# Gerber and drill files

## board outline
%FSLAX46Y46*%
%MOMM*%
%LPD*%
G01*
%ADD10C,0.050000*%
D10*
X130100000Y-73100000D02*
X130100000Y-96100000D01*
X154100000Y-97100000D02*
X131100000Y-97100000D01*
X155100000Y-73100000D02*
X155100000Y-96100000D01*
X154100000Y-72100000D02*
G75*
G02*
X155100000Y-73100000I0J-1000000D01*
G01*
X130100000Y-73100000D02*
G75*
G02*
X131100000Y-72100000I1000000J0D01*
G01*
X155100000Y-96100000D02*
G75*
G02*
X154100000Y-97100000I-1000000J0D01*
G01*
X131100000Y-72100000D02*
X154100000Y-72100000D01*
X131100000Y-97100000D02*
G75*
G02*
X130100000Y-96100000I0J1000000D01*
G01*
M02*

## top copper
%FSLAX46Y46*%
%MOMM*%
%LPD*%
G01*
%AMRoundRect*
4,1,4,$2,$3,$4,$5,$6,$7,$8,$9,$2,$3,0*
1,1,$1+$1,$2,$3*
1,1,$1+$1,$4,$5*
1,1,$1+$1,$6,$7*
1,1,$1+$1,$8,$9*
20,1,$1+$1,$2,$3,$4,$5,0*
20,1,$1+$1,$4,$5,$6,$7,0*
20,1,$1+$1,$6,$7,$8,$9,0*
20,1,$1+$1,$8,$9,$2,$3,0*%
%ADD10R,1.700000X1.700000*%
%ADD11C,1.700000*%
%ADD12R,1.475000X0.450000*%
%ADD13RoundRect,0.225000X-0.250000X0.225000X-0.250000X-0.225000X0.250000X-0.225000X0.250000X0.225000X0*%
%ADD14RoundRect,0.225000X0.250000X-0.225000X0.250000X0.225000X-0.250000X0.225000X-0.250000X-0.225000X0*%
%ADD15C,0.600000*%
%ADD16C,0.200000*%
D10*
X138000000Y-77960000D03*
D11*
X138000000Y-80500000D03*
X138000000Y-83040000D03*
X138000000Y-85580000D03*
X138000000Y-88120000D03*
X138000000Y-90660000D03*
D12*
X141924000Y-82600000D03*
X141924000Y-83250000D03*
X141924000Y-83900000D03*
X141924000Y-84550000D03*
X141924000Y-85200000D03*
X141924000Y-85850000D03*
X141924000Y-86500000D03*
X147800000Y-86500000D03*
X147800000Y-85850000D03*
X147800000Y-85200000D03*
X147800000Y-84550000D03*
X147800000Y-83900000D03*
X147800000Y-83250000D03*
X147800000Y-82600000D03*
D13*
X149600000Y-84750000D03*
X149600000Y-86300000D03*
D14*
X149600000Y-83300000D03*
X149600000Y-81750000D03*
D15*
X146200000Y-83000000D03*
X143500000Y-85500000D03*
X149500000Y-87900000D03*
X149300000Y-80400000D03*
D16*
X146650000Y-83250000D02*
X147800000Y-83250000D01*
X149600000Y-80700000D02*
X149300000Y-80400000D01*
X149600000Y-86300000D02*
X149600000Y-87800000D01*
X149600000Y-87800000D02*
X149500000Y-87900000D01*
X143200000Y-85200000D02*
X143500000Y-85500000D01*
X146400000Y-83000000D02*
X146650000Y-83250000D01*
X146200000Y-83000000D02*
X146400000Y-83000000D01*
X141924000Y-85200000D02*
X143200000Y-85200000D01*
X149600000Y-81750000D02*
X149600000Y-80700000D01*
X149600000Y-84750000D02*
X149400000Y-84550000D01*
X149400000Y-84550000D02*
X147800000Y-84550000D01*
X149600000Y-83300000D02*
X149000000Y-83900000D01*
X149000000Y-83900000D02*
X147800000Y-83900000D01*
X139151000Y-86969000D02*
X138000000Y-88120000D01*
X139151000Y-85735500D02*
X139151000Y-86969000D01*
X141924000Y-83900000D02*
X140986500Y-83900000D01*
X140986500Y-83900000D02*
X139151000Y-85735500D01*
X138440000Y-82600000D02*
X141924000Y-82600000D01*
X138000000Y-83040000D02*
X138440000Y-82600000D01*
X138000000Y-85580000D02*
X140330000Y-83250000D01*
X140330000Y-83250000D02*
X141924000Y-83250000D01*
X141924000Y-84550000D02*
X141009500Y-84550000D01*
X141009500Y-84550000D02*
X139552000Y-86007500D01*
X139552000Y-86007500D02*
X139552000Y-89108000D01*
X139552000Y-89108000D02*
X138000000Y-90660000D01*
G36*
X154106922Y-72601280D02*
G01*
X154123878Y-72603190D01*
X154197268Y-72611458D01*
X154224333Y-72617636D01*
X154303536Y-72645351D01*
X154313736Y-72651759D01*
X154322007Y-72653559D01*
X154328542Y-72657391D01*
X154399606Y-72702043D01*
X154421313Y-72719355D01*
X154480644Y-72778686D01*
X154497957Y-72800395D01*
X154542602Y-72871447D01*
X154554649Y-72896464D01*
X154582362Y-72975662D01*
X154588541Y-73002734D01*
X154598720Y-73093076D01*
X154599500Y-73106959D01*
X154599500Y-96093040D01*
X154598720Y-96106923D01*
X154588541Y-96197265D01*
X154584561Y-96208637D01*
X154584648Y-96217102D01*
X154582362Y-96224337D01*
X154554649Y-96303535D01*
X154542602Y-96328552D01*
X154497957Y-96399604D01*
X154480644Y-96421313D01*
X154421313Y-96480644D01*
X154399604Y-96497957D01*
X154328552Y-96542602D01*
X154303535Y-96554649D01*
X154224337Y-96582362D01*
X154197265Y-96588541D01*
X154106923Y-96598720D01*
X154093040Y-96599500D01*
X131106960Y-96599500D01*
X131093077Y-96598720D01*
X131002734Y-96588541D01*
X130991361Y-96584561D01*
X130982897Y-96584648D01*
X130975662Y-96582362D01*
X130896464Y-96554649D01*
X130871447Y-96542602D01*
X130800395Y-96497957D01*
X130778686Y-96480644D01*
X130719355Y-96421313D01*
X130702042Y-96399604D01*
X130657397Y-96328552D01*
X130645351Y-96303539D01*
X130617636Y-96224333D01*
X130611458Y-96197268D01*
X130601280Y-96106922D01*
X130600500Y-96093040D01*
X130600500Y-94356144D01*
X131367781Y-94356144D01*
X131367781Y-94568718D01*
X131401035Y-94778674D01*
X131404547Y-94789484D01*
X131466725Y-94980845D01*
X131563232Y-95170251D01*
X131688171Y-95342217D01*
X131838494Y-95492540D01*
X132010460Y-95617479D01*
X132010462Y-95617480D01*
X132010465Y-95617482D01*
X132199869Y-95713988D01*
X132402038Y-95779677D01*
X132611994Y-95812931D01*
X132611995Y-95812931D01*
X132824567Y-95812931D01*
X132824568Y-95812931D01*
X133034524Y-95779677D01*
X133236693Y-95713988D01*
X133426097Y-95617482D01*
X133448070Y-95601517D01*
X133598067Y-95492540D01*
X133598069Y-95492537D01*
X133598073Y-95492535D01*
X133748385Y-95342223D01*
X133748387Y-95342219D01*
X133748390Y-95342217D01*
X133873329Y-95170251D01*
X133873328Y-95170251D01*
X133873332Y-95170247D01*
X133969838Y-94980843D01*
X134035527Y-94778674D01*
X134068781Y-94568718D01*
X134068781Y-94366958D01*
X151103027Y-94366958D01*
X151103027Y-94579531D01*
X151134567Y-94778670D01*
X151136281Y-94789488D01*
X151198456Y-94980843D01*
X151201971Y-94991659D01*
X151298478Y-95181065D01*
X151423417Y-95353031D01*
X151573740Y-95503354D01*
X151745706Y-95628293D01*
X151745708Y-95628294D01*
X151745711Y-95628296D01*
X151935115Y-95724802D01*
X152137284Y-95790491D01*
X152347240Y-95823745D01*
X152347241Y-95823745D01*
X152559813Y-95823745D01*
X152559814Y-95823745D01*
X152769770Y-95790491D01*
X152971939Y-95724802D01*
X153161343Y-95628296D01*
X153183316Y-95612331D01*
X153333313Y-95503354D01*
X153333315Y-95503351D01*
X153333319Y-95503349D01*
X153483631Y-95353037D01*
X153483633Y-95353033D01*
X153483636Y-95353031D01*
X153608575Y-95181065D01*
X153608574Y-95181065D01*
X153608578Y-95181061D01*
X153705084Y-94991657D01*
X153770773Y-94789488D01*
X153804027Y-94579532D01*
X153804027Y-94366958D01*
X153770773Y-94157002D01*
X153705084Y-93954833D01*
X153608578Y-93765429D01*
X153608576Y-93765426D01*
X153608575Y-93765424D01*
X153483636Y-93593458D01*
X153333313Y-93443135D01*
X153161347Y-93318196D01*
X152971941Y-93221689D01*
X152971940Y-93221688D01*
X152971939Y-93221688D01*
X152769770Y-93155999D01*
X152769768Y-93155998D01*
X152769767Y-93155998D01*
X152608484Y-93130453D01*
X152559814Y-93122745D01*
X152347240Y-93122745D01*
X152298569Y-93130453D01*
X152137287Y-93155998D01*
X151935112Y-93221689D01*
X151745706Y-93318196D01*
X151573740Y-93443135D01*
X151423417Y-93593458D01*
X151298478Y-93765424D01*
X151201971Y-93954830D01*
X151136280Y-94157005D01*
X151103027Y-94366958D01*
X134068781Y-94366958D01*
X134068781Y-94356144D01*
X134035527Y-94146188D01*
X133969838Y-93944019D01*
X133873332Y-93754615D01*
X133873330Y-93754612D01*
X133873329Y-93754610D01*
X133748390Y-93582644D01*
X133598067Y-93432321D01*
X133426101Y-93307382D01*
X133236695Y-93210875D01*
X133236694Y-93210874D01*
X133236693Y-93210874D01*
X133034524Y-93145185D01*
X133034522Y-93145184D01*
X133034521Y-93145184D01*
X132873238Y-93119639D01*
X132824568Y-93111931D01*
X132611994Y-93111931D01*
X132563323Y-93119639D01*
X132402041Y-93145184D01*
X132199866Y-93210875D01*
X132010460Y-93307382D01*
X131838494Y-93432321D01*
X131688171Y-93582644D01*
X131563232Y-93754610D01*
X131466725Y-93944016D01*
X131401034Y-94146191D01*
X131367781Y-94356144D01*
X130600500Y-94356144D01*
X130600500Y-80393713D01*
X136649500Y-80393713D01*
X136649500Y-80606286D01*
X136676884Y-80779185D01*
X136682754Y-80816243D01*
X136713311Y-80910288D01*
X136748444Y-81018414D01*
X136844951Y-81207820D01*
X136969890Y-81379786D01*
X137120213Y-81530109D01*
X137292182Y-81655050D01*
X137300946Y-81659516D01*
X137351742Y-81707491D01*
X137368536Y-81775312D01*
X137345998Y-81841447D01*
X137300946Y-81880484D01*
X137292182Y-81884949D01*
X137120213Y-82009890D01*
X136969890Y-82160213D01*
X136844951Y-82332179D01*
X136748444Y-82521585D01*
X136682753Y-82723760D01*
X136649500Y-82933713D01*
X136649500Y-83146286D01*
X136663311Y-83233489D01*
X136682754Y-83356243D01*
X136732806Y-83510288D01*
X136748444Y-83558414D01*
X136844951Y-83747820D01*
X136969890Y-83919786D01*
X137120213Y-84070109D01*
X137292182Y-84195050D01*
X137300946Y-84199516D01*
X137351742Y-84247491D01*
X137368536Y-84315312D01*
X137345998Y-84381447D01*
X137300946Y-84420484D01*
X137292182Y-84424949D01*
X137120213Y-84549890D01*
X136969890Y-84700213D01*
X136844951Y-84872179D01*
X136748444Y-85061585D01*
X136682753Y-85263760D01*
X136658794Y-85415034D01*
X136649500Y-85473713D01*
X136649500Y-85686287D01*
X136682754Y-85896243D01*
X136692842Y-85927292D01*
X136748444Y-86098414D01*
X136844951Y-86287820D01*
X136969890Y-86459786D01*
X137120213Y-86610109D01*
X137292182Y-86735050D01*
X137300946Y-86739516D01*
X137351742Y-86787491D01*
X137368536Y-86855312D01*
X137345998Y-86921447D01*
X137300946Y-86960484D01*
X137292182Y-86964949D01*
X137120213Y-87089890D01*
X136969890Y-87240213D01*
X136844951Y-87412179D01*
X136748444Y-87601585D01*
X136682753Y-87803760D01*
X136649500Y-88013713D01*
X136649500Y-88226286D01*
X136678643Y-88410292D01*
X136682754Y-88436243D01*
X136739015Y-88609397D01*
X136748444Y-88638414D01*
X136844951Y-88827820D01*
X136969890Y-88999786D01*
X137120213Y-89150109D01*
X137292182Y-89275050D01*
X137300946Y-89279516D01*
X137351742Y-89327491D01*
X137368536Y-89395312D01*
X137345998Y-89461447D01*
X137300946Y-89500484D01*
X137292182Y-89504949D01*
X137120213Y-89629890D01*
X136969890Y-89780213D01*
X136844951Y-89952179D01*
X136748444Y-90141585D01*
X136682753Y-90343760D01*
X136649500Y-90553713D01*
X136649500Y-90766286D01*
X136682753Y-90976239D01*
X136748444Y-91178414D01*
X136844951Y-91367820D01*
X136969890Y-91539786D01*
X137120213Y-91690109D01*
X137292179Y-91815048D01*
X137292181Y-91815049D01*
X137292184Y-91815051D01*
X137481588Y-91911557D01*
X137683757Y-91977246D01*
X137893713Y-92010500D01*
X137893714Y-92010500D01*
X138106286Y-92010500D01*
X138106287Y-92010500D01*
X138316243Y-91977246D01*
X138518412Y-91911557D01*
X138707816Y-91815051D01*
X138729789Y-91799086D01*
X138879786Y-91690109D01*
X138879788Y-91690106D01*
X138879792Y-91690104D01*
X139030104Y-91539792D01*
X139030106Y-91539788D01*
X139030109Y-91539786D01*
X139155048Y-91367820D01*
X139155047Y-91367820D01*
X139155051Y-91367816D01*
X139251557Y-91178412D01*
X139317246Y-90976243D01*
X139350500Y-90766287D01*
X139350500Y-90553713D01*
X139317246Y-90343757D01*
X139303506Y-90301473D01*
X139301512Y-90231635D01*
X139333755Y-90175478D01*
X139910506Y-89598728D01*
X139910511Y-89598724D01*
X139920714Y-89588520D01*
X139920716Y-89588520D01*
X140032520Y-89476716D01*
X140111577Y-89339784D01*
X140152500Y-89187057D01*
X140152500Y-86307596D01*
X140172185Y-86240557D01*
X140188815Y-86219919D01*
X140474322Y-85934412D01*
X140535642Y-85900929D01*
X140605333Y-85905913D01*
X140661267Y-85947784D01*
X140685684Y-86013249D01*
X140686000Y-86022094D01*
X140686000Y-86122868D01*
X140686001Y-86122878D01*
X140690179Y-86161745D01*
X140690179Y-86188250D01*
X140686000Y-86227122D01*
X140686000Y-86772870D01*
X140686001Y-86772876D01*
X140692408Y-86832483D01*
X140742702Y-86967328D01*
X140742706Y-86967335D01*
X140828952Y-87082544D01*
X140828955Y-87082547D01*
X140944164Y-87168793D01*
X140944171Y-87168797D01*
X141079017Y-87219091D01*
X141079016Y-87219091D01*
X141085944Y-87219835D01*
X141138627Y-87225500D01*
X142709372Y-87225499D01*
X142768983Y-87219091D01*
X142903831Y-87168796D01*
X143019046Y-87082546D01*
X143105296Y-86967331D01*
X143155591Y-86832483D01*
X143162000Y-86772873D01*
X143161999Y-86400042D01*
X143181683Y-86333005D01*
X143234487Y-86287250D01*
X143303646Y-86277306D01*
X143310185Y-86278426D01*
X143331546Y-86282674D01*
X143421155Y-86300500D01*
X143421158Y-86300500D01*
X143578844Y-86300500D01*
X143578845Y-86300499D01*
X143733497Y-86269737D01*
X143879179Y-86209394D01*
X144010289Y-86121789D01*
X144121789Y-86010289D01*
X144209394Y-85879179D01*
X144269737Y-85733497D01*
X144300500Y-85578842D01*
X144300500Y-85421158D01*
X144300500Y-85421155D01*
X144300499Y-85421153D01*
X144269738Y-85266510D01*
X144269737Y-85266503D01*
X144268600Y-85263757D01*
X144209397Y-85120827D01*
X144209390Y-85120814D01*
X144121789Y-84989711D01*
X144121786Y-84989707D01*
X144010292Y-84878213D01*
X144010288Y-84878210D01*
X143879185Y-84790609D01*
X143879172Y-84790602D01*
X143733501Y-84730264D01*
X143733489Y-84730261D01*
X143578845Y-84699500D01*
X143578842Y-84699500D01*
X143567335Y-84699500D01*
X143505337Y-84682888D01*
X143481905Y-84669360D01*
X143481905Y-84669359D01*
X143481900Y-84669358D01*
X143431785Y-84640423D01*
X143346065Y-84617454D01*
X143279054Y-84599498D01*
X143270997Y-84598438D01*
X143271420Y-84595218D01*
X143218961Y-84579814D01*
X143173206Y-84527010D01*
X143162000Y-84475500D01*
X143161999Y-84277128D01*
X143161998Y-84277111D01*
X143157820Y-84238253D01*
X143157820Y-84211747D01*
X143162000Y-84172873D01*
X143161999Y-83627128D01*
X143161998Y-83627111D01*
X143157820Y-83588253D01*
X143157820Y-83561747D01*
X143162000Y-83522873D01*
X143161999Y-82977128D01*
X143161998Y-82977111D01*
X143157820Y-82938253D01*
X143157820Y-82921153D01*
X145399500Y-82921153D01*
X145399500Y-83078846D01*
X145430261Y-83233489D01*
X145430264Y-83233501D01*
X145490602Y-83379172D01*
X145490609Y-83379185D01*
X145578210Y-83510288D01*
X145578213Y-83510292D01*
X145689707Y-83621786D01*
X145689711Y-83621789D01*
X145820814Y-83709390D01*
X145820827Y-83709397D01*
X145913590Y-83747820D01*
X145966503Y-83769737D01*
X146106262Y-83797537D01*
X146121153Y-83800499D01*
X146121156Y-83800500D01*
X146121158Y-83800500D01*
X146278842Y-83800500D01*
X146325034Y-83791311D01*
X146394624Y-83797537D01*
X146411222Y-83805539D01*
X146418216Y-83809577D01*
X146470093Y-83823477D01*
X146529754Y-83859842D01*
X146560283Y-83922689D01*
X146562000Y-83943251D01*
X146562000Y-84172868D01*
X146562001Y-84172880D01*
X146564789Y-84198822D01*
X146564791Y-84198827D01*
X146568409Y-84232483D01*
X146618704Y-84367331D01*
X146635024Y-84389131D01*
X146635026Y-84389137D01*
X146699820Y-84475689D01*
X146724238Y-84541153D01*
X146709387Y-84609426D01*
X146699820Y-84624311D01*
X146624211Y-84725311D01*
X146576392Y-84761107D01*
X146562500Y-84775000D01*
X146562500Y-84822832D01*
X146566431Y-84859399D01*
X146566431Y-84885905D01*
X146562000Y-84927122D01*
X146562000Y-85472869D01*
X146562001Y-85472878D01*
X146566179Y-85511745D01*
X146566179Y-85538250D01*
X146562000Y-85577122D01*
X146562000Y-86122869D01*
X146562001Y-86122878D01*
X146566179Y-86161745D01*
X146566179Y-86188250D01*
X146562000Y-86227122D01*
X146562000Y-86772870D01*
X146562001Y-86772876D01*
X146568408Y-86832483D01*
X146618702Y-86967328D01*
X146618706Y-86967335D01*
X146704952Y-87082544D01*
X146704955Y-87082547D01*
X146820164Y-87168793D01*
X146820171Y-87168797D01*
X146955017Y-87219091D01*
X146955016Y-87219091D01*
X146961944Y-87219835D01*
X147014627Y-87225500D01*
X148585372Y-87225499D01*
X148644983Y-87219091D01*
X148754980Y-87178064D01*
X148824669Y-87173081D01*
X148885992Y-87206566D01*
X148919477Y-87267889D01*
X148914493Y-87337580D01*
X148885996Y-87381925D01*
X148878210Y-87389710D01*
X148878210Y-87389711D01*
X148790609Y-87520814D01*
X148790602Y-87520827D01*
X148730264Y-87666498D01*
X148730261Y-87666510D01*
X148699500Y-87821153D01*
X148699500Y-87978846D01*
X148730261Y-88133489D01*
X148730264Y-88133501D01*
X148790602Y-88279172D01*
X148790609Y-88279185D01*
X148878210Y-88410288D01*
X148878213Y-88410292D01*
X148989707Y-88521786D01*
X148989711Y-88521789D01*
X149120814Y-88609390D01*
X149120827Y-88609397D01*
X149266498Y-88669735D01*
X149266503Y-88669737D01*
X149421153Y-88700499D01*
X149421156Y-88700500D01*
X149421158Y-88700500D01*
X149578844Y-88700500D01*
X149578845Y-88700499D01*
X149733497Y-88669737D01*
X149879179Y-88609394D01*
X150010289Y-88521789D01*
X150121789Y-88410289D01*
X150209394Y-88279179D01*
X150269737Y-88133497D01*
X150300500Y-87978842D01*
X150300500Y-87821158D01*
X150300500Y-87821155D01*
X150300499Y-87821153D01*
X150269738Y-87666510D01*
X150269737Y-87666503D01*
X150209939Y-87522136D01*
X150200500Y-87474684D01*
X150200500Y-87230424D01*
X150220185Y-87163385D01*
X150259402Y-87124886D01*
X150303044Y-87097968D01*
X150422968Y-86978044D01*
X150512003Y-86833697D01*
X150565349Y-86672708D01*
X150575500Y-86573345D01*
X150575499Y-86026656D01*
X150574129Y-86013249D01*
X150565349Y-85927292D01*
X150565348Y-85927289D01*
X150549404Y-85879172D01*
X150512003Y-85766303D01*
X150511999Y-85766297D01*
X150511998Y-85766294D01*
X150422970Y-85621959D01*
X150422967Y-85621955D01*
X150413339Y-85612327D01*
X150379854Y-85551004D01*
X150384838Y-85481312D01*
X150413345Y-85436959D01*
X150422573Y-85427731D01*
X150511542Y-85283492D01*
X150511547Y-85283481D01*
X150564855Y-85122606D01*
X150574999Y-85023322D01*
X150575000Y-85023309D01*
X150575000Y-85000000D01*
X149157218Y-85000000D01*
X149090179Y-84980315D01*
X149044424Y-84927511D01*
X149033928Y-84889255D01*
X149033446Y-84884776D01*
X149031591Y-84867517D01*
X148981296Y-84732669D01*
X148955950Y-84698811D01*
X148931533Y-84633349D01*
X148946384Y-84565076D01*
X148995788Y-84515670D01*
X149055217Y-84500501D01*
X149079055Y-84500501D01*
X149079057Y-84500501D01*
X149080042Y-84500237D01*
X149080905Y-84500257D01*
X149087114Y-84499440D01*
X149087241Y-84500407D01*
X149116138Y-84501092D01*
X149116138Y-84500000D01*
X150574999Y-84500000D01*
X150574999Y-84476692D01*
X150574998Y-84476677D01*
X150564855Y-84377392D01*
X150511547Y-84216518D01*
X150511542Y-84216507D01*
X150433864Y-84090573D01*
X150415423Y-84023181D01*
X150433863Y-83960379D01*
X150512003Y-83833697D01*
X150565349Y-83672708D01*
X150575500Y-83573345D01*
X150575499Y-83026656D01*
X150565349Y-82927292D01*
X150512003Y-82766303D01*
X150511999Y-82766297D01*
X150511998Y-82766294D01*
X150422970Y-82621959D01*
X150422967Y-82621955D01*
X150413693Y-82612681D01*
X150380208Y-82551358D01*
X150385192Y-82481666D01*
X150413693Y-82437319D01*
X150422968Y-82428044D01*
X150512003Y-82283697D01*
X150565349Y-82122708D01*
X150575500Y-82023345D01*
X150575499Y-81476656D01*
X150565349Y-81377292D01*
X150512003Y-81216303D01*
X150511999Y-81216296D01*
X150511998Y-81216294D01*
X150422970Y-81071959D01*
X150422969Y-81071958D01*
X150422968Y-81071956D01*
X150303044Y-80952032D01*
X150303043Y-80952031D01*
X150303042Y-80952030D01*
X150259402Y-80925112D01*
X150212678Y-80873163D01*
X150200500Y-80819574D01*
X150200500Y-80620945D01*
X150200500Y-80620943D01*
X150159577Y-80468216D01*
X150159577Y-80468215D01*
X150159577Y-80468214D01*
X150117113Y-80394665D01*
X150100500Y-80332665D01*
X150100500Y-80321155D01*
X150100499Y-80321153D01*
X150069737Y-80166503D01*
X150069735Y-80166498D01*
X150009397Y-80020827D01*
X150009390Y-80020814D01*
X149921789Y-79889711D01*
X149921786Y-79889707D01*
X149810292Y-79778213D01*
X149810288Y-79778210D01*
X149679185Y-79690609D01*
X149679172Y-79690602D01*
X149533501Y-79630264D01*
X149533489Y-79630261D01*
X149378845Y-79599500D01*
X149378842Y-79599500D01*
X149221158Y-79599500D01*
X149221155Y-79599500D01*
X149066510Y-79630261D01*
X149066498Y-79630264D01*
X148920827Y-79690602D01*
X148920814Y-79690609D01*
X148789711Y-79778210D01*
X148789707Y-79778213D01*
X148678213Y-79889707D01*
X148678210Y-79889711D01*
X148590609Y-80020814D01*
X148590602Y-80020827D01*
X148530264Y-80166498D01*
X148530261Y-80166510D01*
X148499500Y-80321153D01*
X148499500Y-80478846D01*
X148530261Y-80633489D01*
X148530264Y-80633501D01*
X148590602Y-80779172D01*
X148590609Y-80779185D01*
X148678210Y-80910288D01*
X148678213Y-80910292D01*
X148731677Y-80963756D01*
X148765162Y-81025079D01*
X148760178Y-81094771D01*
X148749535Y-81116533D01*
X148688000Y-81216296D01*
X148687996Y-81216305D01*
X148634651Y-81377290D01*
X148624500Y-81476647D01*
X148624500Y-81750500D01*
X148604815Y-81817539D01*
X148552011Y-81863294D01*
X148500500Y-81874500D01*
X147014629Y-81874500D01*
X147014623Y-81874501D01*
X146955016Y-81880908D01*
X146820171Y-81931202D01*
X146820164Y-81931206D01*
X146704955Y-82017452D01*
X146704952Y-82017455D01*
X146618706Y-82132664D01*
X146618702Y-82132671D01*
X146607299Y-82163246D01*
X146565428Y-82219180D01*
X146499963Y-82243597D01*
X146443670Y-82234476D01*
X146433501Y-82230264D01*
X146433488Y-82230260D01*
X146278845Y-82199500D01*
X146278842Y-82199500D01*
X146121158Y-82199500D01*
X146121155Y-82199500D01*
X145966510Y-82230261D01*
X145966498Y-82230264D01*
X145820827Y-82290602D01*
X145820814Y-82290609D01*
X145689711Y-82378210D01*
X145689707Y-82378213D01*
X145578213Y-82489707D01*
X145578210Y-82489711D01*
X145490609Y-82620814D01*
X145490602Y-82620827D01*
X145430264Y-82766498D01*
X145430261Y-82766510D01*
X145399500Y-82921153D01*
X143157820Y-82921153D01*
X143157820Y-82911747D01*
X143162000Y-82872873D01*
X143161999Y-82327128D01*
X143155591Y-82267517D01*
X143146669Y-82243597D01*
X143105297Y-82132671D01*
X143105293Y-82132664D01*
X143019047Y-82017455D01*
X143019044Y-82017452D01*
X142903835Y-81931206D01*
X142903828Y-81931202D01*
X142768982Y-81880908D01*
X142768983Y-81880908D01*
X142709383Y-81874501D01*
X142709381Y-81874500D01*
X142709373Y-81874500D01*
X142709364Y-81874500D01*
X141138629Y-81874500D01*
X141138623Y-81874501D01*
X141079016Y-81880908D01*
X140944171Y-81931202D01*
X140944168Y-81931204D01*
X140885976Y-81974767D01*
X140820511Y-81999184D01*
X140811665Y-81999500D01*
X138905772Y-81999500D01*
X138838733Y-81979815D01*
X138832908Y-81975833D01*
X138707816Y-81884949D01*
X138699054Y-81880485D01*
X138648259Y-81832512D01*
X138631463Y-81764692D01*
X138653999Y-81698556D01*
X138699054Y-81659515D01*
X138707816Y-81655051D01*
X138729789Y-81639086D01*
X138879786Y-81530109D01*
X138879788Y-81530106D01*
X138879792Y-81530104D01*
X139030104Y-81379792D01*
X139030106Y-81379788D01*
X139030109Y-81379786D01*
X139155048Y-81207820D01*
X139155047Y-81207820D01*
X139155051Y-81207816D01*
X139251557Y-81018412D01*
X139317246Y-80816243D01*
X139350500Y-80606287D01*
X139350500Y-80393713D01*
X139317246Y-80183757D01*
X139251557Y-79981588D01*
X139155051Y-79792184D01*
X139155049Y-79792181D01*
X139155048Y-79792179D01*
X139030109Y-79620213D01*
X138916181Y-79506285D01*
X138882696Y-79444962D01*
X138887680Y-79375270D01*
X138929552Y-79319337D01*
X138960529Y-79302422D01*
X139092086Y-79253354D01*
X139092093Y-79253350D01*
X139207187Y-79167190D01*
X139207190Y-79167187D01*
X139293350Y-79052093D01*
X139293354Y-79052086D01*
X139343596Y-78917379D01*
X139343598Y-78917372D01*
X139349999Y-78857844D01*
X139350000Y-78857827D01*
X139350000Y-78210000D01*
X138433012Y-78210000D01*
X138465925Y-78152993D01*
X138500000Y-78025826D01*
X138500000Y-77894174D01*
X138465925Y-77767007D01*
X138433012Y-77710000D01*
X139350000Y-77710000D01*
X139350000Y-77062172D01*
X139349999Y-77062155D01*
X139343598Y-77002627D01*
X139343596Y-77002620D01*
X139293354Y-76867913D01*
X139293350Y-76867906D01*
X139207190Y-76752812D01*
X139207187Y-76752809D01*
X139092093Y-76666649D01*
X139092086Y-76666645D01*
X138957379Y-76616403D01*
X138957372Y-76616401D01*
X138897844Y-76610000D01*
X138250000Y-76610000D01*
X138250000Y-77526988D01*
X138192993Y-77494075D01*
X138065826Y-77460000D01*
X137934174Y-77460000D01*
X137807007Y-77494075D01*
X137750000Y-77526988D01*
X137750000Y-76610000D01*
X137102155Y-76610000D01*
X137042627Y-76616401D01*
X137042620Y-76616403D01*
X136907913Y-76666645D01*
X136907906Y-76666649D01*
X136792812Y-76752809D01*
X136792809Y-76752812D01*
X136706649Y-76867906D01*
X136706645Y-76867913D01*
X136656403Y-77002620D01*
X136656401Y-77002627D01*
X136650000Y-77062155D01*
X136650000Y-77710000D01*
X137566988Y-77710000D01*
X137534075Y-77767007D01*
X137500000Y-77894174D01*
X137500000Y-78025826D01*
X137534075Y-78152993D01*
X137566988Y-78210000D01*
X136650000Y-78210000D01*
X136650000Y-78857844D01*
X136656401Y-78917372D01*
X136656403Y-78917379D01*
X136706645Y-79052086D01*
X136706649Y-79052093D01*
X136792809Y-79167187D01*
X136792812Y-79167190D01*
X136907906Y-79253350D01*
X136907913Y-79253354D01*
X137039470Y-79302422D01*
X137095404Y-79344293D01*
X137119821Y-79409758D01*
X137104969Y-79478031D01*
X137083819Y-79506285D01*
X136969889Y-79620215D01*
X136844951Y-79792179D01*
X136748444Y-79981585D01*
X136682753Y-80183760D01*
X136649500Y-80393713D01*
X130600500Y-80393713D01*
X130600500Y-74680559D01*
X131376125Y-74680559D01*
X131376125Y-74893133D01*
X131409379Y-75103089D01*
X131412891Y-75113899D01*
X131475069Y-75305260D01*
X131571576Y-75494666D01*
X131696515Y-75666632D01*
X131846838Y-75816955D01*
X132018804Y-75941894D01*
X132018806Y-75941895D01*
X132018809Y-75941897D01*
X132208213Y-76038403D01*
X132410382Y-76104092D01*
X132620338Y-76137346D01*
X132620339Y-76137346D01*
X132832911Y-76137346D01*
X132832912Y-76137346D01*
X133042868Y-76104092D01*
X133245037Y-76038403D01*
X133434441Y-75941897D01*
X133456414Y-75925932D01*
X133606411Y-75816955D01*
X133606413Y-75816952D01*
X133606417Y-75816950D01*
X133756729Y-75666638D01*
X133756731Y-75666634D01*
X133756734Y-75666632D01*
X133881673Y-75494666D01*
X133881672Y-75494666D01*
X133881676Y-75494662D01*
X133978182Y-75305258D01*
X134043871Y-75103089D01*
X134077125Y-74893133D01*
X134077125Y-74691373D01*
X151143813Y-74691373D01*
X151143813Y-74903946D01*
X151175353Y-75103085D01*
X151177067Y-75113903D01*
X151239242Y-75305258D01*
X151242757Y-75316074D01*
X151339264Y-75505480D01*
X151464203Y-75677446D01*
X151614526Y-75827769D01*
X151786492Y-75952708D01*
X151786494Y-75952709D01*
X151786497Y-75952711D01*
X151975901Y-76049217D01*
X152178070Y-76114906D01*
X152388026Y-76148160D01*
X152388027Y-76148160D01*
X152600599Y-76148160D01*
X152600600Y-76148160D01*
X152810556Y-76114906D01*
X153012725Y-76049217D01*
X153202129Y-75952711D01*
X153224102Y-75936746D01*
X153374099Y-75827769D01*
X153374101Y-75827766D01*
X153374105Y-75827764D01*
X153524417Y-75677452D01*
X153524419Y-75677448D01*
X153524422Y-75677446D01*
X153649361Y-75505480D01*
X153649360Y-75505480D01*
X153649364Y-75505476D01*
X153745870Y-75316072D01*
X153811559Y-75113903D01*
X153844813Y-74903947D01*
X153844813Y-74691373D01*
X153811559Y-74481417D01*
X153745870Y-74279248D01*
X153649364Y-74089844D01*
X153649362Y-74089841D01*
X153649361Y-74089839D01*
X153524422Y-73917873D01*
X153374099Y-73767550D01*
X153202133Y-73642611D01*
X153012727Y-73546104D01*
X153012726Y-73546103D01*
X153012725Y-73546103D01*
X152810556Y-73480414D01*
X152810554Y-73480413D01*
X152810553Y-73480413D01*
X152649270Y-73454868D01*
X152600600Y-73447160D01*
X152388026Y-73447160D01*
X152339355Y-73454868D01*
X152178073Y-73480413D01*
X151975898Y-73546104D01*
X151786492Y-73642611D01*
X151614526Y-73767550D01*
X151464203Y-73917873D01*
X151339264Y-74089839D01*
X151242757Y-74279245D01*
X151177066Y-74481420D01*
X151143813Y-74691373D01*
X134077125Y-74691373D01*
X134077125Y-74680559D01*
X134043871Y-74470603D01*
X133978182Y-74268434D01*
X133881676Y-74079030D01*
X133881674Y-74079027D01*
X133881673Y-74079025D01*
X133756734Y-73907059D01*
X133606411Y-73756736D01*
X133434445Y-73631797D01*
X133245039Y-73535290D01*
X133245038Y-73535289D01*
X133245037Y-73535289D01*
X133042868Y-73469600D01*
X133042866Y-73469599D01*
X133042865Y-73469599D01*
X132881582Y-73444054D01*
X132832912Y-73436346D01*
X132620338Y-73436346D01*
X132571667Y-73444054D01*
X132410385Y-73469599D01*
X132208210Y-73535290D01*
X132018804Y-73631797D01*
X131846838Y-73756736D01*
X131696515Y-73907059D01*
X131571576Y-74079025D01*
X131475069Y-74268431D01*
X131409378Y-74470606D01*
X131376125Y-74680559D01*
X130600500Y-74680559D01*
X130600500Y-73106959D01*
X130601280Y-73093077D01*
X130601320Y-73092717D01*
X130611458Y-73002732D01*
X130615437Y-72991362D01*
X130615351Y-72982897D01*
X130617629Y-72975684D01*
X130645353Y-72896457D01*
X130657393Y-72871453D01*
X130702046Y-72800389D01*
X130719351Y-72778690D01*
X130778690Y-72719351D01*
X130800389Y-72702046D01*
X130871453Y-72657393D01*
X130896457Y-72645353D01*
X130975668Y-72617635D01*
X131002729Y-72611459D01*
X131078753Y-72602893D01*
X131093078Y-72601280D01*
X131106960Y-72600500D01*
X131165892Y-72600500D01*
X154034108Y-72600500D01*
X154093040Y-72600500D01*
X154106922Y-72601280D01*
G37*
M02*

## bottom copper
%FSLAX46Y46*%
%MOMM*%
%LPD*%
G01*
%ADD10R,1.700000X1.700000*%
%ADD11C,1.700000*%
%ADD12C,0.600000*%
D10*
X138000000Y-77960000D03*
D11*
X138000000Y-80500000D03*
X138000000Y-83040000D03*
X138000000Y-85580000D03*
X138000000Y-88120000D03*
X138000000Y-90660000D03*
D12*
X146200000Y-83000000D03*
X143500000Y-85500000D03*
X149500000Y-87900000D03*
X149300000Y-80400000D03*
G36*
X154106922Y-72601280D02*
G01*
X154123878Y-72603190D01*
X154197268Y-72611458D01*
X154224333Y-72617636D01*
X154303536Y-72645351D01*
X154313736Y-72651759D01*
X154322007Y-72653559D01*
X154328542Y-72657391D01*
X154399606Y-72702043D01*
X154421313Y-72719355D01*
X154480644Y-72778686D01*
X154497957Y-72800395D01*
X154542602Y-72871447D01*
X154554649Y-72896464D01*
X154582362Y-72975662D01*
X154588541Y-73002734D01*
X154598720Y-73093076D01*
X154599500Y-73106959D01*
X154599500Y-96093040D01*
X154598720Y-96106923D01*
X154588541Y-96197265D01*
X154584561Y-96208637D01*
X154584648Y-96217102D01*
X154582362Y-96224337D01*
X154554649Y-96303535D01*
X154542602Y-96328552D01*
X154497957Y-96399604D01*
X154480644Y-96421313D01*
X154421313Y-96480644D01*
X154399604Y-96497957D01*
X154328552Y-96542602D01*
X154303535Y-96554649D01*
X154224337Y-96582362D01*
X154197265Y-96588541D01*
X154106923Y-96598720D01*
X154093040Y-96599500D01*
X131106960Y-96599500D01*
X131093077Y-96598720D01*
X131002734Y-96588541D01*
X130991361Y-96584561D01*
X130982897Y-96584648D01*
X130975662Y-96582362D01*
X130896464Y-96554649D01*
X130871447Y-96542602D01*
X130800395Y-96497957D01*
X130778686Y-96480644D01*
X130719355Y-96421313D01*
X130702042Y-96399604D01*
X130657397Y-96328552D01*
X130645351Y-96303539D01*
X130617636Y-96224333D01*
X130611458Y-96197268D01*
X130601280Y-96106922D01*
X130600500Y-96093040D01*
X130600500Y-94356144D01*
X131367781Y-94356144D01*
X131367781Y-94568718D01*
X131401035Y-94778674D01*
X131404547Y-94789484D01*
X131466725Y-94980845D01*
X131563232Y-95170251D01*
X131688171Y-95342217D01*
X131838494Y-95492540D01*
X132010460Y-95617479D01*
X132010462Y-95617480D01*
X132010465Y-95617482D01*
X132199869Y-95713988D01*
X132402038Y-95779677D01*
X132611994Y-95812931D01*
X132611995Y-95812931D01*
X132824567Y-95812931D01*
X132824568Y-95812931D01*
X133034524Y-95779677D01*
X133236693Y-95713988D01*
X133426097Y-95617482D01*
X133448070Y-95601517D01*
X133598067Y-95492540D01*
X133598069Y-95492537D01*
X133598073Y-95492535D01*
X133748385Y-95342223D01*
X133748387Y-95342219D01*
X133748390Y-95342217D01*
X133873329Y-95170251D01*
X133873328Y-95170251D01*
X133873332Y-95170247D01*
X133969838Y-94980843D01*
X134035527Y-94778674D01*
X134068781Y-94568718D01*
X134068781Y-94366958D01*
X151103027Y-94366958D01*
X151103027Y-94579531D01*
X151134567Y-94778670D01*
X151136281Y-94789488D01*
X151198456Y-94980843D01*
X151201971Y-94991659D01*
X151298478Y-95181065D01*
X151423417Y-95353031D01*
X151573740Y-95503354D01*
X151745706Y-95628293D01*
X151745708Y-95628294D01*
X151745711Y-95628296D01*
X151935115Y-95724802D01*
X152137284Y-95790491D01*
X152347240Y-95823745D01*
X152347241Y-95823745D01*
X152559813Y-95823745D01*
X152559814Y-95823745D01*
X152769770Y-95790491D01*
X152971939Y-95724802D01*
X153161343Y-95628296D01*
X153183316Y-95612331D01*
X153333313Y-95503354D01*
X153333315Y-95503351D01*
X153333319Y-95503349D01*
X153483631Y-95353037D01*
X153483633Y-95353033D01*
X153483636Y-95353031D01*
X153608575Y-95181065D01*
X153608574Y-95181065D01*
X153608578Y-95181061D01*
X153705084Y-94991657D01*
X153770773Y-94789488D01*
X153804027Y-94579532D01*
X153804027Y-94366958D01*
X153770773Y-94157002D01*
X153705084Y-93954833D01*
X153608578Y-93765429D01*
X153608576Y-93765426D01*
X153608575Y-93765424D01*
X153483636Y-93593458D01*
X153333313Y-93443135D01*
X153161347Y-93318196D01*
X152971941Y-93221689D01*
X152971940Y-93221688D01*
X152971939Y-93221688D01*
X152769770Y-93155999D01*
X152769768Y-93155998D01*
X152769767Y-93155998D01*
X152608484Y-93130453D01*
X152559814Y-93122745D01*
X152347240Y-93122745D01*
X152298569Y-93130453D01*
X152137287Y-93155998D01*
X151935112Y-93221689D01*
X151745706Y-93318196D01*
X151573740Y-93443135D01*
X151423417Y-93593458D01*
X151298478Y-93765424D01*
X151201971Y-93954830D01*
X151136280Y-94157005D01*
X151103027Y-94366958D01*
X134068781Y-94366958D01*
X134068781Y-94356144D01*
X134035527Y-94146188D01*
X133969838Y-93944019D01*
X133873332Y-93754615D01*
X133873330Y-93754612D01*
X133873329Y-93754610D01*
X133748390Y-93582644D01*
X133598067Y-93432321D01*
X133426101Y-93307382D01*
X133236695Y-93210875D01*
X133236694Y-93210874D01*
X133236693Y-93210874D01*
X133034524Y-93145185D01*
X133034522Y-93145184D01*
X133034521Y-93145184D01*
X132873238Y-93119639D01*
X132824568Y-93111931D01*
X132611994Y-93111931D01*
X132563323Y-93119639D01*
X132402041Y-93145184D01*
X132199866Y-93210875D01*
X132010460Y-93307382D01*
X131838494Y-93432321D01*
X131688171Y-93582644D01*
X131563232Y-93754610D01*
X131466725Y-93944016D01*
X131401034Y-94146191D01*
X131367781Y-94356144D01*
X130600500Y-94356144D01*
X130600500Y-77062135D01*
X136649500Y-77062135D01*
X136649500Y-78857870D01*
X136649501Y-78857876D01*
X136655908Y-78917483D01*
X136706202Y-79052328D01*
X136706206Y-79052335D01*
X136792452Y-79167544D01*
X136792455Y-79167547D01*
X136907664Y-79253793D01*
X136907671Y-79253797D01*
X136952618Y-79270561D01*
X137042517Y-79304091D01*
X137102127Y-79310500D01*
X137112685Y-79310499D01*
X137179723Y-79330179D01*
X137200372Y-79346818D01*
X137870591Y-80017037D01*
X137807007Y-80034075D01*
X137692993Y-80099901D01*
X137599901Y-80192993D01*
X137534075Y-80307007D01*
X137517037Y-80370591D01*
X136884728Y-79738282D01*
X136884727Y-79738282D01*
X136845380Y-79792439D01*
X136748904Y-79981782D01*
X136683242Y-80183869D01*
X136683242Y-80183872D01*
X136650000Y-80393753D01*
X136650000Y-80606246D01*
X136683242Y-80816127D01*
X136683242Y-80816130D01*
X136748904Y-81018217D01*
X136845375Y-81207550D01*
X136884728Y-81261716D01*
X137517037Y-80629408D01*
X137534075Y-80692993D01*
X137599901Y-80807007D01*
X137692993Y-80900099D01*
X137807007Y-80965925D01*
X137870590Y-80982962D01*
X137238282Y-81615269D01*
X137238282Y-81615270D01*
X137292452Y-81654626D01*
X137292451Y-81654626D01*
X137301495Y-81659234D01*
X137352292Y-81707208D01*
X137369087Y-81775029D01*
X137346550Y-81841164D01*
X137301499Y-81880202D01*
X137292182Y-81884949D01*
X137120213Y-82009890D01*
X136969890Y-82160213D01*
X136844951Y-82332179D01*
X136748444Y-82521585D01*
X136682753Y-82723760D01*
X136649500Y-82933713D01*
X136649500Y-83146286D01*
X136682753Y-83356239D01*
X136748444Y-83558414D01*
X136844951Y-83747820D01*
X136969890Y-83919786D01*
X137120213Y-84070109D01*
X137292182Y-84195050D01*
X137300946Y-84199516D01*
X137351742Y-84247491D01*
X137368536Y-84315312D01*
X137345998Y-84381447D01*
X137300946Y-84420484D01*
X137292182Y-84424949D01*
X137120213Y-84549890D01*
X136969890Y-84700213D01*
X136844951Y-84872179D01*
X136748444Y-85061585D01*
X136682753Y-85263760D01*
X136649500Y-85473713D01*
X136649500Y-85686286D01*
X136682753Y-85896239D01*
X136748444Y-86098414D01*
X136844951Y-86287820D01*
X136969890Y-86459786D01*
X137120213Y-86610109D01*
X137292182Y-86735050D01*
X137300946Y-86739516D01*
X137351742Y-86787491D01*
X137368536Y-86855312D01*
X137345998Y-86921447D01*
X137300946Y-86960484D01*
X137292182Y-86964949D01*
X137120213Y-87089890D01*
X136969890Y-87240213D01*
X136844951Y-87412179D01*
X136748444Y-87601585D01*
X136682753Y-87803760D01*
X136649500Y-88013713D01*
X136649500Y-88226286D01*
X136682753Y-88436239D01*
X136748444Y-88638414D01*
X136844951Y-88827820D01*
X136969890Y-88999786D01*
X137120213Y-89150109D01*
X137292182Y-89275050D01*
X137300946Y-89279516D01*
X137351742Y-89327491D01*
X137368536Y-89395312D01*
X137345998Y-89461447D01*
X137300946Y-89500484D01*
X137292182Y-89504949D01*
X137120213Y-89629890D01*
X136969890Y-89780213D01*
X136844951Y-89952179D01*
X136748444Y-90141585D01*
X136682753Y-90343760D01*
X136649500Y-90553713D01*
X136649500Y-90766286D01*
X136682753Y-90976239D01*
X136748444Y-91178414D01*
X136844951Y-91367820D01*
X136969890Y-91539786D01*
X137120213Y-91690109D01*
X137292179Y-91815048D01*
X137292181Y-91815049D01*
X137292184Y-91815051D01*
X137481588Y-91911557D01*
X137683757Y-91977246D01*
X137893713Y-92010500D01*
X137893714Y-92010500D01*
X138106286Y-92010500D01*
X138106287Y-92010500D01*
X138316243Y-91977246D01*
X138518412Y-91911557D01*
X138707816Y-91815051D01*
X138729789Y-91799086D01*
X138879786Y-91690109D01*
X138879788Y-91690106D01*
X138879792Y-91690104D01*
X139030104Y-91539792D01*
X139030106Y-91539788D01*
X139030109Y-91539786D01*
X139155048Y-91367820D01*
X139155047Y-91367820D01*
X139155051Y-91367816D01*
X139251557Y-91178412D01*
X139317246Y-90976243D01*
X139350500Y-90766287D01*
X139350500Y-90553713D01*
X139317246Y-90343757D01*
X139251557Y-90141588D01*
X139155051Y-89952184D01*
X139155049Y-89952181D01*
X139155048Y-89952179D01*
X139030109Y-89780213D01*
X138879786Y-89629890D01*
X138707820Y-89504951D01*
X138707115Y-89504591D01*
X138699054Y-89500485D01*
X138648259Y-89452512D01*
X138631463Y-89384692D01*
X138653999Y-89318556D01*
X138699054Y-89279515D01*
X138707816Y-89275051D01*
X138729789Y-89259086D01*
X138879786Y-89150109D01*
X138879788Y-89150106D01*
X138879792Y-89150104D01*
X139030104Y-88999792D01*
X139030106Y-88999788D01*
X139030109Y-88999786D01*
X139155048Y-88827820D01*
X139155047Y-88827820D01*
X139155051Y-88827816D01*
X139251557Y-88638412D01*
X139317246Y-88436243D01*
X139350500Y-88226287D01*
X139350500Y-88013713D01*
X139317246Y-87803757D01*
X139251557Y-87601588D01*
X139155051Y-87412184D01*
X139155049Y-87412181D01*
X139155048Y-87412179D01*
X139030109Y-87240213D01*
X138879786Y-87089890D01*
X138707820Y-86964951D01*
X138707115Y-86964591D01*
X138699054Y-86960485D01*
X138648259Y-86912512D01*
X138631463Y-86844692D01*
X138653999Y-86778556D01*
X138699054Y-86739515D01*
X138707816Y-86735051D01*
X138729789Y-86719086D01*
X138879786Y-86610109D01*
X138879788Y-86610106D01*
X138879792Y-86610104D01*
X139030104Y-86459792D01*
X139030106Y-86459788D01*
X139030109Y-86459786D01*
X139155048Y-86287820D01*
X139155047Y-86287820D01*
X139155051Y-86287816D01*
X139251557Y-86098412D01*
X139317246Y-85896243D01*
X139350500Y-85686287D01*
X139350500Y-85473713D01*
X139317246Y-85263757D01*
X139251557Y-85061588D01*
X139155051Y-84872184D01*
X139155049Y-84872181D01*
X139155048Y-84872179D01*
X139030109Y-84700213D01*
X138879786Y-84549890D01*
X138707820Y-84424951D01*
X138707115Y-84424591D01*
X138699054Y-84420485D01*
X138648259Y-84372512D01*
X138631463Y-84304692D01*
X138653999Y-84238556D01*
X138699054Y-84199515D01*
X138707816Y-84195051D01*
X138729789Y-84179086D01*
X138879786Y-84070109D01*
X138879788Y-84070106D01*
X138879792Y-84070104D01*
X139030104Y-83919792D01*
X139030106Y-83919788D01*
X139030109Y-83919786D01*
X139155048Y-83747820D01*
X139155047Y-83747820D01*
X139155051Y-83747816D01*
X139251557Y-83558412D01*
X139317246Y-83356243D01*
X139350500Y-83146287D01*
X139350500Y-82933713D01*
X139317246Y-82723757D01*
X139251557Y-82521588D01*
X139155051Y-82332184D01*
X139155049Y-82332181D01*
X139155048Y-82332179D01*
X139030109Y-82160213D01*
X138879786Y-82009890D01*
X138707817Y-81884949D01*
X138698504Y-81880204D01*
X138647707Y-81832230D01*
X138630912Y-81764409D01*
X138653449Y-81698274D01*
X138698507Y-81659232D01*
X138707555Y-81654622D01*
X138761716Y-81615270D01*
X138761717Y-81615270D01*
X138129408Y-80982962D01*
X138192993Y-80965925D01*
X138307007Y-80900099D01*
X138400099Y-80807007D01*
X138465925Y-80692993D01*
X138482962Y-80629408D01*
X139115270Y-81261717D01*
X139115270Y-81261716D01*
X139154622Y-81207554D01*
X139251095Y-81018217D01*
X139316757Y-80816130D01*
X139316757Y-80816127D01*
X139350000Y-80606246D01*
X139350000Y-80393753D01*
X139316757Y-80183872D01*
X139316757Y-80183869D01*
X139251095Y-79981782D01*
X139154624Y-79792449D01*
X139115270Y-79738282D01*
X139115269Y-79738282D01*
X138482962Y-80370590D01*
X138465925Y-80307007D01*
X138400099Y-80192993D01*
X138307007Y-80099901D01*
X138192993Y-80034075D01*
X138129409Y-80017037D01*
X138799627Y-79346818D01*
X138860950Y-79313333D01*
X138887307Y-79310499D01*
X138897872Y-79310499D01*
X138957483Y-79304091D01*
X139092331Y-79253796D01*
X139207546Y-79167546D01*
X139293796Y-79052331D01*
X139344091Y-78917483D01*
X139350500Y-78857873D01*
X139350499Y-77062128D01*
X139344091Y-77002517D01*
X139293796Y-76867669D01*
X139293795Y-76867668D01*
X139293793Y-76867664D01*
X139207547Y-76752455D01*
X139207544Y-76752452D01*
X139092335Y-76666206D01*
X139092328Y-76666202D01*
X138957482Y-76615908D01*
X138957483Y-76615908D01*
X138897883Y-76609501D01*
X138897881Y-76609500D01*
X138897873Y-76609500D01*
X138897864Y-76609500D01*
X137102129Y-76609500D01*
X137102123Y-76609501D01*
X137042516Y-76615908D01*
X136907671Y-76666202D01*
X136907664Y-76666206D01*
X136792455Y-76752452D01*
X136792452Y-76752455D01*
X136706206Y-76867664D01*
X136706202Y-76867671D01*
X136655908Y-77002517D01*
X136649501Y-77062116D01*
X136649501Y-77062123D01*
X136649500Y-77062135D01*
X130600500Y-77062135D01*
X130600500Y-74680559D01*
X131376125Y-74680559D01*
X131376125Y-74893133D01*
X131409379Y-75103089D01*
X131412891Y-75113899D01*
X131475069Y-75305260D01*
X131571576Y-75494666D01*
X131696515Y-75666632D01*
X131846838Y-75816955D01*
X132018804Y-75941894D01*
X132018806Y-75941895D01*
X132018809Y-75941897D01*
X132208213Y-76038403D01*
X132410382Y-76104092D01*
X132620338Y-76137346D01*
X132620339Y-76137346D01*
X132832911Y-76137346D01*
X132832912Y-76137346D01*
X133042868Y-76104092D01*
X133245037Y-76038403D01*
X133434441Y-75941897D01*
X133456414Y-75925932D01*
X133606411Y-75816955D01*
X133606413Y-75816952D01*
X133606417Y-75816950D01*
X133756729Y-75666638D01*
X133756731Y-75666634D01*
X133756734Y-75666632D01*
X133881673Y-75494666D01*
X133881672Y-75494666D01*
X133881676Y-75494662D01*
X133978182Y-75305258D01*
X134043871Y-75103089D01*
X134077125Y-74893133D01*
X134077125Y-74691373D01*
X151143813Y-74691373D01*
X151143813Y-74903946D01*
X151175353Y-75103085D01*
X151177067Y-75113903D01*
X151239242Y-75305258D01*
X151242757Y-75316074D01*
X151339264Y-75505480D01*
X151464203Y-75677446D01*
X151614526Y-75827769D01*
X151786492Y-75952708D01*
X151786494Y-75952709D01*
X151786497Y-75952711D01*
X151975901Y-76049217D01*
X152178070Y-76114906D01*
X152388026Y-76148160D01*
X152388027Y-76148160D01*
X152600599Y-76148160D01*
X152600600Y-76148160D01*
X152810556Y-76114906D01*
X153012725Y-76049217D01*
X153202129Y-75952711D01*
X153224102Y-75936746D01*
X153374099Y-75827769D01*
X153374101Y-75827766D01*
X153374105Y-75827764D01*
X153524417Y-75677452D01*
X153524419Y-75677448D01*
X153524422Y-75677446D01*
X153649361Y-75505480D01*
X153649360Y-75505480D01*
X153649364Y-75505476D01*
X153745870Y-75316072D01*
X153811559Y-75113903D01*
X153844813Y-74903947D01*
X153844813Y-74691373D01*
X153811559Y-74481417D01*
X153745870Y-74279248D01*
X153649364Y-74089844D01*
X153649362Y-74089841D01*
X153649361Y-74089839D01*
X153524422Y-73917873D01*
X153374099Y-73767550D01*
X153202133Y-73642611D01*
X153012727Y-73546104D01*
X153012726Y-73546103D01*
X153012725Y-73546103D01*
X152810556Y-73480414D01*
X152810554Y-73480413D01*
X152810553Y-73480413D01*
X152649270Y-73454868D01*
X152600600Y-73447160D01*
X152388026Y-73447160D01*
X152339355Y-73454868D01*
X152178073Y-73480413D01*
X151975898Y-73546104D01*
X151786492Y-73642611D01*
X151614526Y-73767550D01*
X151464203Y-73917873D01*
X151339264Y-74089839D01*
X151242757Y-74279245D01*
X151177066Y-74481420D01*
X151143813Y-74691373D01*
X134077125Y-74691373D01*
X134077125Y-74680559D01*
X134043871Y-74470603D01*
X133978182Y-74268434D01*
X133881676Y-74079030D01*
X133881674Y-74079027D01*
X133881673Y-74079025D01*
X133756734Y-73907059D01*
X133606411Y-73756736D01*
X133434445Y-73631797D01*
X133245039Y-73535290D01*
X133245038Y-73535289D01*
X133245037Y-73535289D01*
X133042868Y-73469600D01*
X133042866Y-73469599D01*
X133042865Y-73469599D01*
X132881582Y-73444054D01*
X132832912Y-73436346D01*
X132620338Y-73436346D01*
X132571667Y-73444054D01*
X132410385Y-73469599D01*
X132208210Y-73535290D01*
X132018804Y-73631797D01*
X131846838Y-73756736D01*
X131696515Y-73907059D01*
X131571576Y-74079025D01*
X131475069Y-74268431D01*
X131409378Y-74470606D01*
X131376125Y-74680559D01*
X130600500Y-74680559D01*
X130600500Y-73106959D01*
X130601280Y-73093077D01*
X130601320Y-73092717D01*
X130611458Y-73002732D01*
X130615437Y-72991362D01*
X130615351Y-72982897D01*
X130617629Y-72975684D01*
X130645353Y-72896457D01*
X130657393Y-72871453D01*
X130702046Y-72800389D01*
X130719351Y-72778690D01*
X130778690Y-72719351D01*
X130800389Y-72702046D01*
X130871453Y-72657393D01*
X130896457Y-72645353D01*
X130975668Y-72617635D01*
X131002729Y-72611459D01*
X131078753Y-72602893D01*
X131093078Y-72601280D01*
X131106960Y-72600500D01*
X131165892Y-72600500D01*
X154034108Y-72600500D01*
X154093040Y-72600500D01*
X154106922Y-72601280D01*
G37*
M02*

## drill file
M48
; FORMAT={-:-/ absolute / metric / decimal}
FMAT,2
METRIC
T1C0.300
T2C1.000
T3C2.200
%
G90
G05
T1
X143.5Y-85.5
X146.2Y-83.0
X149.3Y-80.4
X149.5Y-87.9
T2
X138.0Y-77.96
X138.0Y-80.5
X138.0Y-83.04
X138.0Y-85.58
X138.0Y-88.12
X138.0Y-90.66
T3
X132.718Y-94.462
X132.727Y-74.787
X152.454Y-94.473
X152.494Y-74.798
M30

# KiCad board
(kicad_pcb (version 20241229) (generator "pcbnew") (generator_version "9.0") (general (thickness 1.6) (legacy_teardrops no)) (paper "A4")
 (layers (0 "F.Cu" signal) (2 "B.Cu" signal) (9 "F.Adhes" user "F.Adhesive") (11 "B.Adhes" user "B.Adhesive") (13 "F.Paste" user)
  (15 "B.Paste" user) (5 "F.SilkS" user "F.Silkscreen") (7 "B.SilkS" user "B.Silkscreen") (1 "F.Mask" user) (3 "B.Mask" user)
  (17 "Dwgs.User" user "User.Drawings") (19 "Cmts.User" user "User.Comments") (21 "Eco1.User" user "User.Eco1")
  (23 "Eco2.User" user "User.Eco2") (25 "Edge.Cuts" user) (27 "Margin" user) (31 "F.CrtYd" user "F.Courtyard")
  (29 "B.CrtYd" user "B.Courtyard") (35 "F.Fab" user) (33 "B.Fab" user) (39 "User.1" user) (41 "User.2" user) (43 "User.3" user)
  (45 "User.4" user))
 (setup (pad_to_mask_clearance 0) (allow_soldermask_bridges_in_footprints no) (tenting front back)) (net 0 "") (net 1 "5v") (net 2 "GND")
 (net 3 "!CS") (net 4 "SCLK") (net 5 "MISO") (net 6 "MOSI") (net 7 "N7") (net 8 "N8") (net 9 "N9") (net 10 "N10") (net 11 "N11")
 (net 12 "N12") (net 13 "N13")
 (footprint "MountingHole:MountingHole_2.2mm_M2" (layer "F.Cu") (at 152.494313 74.79766)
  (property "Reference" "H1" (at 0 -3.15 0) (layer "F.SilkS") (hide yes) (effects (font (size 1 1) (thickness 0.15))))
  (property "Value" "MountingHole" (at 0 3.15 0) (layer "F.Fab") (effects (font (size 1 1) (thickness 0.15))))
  (pad "" np_thru_hole circle (at 0 0) (size 2.2 2.2) (drill 2.2) (layers "*.Cu" "*.Mask")))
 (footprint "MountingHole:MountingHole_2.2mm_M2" (layer "F.Cu") (at 152.453527 94.473245)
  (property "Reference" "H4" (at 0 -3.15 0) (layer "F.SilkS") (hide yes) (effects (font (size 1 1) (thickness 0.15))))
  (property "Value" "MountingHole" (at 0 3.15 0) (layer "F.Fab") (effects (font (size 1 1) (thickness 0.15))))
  (pad "" np_thru_hole circle (at 0 0) (size 2.2 2.2) (drill 2.2) (layers "*.Cu" "*.Mask")))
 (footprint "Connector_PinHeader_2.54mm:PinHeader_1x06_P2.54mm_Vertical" (layer "F.Cu") (at 138 77.96)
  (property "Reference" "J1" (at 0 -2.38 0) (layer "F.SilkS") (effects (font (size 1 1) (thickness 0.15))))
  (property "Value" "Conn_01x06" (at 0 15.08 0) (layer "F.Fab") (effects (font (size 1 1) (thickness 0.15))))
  (pad "1" thru_hole rect (at 0 0) (size 1.7 1.7) (drill 1) (layers "*.Cu" "*.Mask") (remove_unused_layers no) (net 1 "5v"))
  (pad "2" thru_hole circle (at 0 2.54) (size 1.7 1.7) (drill 1) (layers "*.Cu" "*.Mask") (remove_unused_layers no) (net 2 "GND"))
  (pad "3" thru_hole circle (at 0 5.08) (size 1.7 1.7) (drill 1) (layers "*.Cu" "*.Mask") (remove_unused_layers no) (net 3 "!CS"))
  (pad "4" thru_hole circle (at 0 7.62) (size 1.7 1.7) (drill 1) (layers "*.Cu" "*.Mask") (remove_unused_layers no) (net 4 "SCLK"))
  (pad "5" thru_hole circle (at 0 10.16) (size 1.7 1.7) (drill 1) (layers "*.Cu" "*.Mask") (remove_unused_layers no) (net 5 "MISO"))
  (pad "6" thru_hole circle (at 0 12.7) (size 1.7 1.7) (drill 1) (layers "*.Cu" "*.Mask") (remove_unused_layers no) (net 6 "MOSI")))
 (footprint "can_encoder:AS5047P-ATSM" (layer "F.Cu") (at 144.862 84.55)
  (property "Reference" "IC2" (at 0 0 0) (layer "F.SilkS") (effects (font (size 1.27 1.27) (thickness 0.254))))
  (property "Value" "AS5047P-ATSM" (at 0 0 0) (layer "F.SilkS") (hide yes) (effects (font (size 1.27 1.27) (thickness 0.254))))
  (pad "1" smd rect (at -2.938 -1.95 90) (size 0.45 1.475) (layers "F.Cu" "F.Mask" "F.Paste") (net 3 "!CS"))
  (pad "2" smd rect (at -2.938 -1.3 90) (size 0.45 1.475) (layers "F.Cu" "F.Mask" "F.Paste") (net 4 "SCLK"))
  (pad "3" smd rect (at -2.938 -0.65 90) (size 0.45 1.475) (layers "F.Cu" "F.Mask" "F.Paste") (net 5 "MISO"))
  (pad "4" smd rect (at -2.938 0 90) (size 0.45 1.475) (layers "F.Cu" "F.Mask" "F.Paste") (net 6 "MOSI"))
  (pad "5" smd rect (at -2.938 0.65 90) (size 0.45 1.475) (layers "F.Cu" "F.Mask" "F.Paste") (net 2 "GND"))
  (pad "6" smd rect (at -2.938 1.3 90) (size 0.45 1.475) (layers "F.Cu" "F.Mask" "F.Paste") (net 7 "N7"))
  (pad "7" smd rect (at -2.938 1.95 90) (size 0.45 1.475) (layers "F.Cu" "F.Mask" "F.Paste") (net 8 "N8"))
  (pad "8" smd rect (at 2.938 1.95 90) (size 0.45 1.475) (layers "F.Cu" "F.Mask" "F.Paste") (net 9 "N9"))
  (pad "9" smd rect (at 2.938 1.3 90) (size 0.45 1.475) (layers "F.Cu" "F.Mask" "F.Paste") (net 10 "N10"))
  (pad "10" smd rect (at 2.938 0.65 90) (size 0.45 1.475) (layers "F.Cu" "F.Mask" "F.Paste") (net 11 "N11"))
  (pad "11" smd rect (at 2.938 0 90) (size 0.45 1.475) (layers "F.Cu" "F.Mask" "F.Paste") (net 1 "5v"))
  (pad "12" smd rect (at 2.938 -0.65 90) (size 0.45 1.475) (layers "F.Cu" "F.Mask" "F.Paste") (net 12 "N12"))
  (pad "13" smd rect (at 2.938 -1.3 90) (size 0.45 1.475) (layers "F.Cu" "F.Mask" "F.Paste") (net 2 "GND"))
  (pad "14" smd rect (at 2.938 -1.95 90) (size 0.45 1.475) (layers "F.Cu" "F.Mask" "F.Paste") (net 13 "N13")))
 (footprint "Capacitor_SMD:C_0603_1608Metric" (layer "F.Cu") (at 149.6 85.525 -90)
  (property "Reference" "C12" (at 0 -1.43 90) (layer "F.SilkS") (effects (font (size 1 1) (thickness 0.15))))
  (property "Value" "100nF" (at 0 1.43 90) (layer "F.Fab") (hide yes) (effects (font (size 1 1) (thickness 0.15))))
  (pad "1" smd roundrect (at -0.775 0 270) (size 0.9 0.95) (layers "F.Cu" "F.Mask" "F.Paste") (roundrect_rratio 0.25) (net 1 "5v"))
  (pad "2" smd roundrect (at 0.775 0 270) (size 0.9 0.95) (layers "F.Cu" "F.Mask" "F.Paste") (roundrect_rratio 0.25) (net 2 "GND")))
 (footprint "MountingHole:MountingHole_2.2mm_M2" (layer "F.Cu") (at 132.726625 74.786846)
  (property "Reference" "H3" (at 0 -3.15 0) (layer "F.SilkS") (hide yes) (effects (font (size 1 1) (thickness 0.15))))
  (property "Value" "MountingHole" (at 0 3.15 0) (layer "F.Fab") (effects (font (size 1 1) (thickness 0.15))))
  (pad "" np_thru_hole circle (at 0 0) (size 2.2 2.2) (drill 2.2) (layers "*.Cu" "*.Mask")))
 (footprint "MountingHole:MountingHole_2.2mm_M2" (layer "F.Cu") (at 132.718281 94.462431)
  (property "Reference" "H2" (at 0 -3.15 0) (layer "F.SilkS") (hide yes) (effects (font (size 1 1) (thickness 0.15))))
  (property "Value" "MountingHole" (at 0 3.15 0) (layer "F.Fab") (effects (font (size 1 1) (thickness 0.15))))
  (pad "" np_thru_hole circle (at 0 0) (size 2.2 2.2) (drill 2.2) (layers "*.Cu" "*.Mask")))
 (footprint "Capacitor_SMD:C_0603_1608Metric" (layer "F.Cu") (at 149.6 82.525 90)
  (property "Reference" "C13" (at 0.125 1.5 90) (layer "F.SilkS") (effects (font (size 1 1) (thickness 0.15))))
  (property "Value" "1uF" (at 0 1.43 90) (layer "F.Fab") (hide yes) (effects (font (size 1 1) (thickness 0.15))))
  (pad "1" smd roundrect (at -0.775 0 90) (size 0.9 0.95) (layers "F.Cu" "F.Mask" "F.Paste") (roundrect_rratio 0.25) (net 12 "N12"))
  (pad "2" smd roundrect (at 0.775 0 90) (size 0.9 0.95) (layers "F.Cu" "F.Mask" "F.Paste") (roundrect_rratio 0.25) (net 2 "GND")))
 (gr_line (start 130.1 73.1) (end 130.1 96.1) (stroke (width 0.05) (type default)) (layer "Edge.Cuts"))
 (gr_line (start 154.1 97.1) (end 131.1 97.1) (stroke (width 0.05) (type default)) (layer "Edge.Cuts"))
 (gr_line (start 155.1 73.1) (end 155.1 96.1) (stroke (width 0.05) (type default)) (layer "Edge.Cuts"))
 (gr_arc (start 154.1 72.1) (mid 154.807107 72.392893) (end 155.1 73.1) (stroke (width 0.05) (type default)) (layer "Edge.Cuts"))
 (gr_arc (start 130.1 73.1) (mid 130.392893 72.392893) (end 131.1 72.1) (stroke (width 0.05) (type default)) (layer "Edge.Cuts"))
 (gr_arc (start 155.1 96.1) (mid 154.807107 96.807107) (end 154.1 97.1) (stroke (width 0.05) (type default)) (layer "Edge.Cuts"))
 (gr_line (start 131.1 72.1) (end 154.1 72.1) (stroke (width 0.05) (type default)) (layer "Edge.Cuts"))
 (gr_arc (start 131.1 97.1) (mid 130.392893 96.807107) (end 130.1 96.1) (stroke (width 0.05) (type default)) (layer "Edge.Cuts"))
 (segment (start 146.65 83.25) (end 147.8 83.25) (width 0.2) (layer "F.Cu") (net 2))
 (segment (start 149.6 80.7) (end 149.3 80.4) (width 0.2) (layer "F.Cu") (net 2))
 (segment (start 149.6 86.3) (end 149.6 87.8) (width 0.2) (layer "F.Cu") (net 2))
 (segment (start 149.6 87.8) (end 149.5 87.9) (width 0.2) (layer "F.Cu") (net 2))
 (segment (start 143.2 85.2) (end 143.5 85.5) (width 0.2) (layer "F.Cu") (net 2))
 (segment (start 146.4 83) (end 146.65 83.25) (width 0.2) (layer "F.Cu") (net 2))
 (segment (start 146.2 83) (end 146.4 83) (width 0.2) (layer "F.Cu") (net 2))
 (segment (start 141.924 85.2) (end 143.2 85.2) (width 0.2) (layer "F.Cu") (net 2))
 (segment (start 149.6 81.75) (end 149.6 80.7) (width 0.2) (layer "F.Cu") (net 2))
 (via (at 146.2 83) (size 0.6) (drill 0.3) (layers "F.Cu" "B.Cu") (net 2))
 (via (at 143.5 85.5) (size 0.6) (drill 0.3) (layers "F.Cu" "B.Cu") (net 2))
 (via (at 149.5 87.9) (size 0.6) (drill 0.3) (layers "F.Cu" "B.Cu") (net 2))
 (via (at 149.3 80.4) (size 0.6) (drill 0.3) (layers "F.Cu" "B.Cu") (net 2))
 (segment (start 149.6 84.75) (end 149.4 84.55) (width 0.2) (layer "F.Cu") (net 1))
 (segment (start 149.4 84.55) (end 147.8 84.55) (width 0.2) (layer "F.Cu") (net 1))
 (segment (start 149.6 83.3) (end 149 83.9) (width 0.2) (layer "F.Cu") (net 12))
 (segment (start 149 83.9) (end 147.8 83.9) (width 0.2) (layer "F.Cu") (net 12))
 (segment (start 139.151 86.969) (end 138 88.12) (width 0.2) (layer "F.Cu") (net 5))
 (segment (start 139.151 85.7355) (end 139.151 86.969) (width 0.2) (layer "F.Cu") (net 5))
 (segment (start 141.924 83.9) (end 140.9865 83.9) (width 0.2) (layer "F.Cu") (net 5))
 (segment (start 140.9865 83.9) (end 139.151 85.7355) (width 0.2) (layer "F.Cu") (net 5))
 (segment (start 138.44 82.6) (end 141.924 82.6) (width 0.2) (layer "F.Cu") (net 3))
 (segment (start 138 83.04) (end 138.44 82.6) (width 0.2) (layer "F.Cu") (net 3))
 (segment (start 138 85.58) (end 140.33 83.25) (width 0.2) (layer "F.Cu") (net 4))
 (segment (start 140.33 83.25) (end 141.924 83.25) (width 0.2) (layer "F.Cu") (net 4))
 (segment (start 141.924 84.55) (end 141.0095 84.55) (width 0.2) (layer "F.Cu") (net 6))
 (segment (start 141.0095 84.55) (end 139.552 86.0075) (width 0.2) (layer "F.Cu") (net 6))
 (segment (start 139.552 86.0075) (end 139.552 89.108) (width 0.2) (layer "F.Cu") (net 6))
 (segment (start 139.552 89.108) (end 138 90.66) (width 0.2) (layer "F.Cu") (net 6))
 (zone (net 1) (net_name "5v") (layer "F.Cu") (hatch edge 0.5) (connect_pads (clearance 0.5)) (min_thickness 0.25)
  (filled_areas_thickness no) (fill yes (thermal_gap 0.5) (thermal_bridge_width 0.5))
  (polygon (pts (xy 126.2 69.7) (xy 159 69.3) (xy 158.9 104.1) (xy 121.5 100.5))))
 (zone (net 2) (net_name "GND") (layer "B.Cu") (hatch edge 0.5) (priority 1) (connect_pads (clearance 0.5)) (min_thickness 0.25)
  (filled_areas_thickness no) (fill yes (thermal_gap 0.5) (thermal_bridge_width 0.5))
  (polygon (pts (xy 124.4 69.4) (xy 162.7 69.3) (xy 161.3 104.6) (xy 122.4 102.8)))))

